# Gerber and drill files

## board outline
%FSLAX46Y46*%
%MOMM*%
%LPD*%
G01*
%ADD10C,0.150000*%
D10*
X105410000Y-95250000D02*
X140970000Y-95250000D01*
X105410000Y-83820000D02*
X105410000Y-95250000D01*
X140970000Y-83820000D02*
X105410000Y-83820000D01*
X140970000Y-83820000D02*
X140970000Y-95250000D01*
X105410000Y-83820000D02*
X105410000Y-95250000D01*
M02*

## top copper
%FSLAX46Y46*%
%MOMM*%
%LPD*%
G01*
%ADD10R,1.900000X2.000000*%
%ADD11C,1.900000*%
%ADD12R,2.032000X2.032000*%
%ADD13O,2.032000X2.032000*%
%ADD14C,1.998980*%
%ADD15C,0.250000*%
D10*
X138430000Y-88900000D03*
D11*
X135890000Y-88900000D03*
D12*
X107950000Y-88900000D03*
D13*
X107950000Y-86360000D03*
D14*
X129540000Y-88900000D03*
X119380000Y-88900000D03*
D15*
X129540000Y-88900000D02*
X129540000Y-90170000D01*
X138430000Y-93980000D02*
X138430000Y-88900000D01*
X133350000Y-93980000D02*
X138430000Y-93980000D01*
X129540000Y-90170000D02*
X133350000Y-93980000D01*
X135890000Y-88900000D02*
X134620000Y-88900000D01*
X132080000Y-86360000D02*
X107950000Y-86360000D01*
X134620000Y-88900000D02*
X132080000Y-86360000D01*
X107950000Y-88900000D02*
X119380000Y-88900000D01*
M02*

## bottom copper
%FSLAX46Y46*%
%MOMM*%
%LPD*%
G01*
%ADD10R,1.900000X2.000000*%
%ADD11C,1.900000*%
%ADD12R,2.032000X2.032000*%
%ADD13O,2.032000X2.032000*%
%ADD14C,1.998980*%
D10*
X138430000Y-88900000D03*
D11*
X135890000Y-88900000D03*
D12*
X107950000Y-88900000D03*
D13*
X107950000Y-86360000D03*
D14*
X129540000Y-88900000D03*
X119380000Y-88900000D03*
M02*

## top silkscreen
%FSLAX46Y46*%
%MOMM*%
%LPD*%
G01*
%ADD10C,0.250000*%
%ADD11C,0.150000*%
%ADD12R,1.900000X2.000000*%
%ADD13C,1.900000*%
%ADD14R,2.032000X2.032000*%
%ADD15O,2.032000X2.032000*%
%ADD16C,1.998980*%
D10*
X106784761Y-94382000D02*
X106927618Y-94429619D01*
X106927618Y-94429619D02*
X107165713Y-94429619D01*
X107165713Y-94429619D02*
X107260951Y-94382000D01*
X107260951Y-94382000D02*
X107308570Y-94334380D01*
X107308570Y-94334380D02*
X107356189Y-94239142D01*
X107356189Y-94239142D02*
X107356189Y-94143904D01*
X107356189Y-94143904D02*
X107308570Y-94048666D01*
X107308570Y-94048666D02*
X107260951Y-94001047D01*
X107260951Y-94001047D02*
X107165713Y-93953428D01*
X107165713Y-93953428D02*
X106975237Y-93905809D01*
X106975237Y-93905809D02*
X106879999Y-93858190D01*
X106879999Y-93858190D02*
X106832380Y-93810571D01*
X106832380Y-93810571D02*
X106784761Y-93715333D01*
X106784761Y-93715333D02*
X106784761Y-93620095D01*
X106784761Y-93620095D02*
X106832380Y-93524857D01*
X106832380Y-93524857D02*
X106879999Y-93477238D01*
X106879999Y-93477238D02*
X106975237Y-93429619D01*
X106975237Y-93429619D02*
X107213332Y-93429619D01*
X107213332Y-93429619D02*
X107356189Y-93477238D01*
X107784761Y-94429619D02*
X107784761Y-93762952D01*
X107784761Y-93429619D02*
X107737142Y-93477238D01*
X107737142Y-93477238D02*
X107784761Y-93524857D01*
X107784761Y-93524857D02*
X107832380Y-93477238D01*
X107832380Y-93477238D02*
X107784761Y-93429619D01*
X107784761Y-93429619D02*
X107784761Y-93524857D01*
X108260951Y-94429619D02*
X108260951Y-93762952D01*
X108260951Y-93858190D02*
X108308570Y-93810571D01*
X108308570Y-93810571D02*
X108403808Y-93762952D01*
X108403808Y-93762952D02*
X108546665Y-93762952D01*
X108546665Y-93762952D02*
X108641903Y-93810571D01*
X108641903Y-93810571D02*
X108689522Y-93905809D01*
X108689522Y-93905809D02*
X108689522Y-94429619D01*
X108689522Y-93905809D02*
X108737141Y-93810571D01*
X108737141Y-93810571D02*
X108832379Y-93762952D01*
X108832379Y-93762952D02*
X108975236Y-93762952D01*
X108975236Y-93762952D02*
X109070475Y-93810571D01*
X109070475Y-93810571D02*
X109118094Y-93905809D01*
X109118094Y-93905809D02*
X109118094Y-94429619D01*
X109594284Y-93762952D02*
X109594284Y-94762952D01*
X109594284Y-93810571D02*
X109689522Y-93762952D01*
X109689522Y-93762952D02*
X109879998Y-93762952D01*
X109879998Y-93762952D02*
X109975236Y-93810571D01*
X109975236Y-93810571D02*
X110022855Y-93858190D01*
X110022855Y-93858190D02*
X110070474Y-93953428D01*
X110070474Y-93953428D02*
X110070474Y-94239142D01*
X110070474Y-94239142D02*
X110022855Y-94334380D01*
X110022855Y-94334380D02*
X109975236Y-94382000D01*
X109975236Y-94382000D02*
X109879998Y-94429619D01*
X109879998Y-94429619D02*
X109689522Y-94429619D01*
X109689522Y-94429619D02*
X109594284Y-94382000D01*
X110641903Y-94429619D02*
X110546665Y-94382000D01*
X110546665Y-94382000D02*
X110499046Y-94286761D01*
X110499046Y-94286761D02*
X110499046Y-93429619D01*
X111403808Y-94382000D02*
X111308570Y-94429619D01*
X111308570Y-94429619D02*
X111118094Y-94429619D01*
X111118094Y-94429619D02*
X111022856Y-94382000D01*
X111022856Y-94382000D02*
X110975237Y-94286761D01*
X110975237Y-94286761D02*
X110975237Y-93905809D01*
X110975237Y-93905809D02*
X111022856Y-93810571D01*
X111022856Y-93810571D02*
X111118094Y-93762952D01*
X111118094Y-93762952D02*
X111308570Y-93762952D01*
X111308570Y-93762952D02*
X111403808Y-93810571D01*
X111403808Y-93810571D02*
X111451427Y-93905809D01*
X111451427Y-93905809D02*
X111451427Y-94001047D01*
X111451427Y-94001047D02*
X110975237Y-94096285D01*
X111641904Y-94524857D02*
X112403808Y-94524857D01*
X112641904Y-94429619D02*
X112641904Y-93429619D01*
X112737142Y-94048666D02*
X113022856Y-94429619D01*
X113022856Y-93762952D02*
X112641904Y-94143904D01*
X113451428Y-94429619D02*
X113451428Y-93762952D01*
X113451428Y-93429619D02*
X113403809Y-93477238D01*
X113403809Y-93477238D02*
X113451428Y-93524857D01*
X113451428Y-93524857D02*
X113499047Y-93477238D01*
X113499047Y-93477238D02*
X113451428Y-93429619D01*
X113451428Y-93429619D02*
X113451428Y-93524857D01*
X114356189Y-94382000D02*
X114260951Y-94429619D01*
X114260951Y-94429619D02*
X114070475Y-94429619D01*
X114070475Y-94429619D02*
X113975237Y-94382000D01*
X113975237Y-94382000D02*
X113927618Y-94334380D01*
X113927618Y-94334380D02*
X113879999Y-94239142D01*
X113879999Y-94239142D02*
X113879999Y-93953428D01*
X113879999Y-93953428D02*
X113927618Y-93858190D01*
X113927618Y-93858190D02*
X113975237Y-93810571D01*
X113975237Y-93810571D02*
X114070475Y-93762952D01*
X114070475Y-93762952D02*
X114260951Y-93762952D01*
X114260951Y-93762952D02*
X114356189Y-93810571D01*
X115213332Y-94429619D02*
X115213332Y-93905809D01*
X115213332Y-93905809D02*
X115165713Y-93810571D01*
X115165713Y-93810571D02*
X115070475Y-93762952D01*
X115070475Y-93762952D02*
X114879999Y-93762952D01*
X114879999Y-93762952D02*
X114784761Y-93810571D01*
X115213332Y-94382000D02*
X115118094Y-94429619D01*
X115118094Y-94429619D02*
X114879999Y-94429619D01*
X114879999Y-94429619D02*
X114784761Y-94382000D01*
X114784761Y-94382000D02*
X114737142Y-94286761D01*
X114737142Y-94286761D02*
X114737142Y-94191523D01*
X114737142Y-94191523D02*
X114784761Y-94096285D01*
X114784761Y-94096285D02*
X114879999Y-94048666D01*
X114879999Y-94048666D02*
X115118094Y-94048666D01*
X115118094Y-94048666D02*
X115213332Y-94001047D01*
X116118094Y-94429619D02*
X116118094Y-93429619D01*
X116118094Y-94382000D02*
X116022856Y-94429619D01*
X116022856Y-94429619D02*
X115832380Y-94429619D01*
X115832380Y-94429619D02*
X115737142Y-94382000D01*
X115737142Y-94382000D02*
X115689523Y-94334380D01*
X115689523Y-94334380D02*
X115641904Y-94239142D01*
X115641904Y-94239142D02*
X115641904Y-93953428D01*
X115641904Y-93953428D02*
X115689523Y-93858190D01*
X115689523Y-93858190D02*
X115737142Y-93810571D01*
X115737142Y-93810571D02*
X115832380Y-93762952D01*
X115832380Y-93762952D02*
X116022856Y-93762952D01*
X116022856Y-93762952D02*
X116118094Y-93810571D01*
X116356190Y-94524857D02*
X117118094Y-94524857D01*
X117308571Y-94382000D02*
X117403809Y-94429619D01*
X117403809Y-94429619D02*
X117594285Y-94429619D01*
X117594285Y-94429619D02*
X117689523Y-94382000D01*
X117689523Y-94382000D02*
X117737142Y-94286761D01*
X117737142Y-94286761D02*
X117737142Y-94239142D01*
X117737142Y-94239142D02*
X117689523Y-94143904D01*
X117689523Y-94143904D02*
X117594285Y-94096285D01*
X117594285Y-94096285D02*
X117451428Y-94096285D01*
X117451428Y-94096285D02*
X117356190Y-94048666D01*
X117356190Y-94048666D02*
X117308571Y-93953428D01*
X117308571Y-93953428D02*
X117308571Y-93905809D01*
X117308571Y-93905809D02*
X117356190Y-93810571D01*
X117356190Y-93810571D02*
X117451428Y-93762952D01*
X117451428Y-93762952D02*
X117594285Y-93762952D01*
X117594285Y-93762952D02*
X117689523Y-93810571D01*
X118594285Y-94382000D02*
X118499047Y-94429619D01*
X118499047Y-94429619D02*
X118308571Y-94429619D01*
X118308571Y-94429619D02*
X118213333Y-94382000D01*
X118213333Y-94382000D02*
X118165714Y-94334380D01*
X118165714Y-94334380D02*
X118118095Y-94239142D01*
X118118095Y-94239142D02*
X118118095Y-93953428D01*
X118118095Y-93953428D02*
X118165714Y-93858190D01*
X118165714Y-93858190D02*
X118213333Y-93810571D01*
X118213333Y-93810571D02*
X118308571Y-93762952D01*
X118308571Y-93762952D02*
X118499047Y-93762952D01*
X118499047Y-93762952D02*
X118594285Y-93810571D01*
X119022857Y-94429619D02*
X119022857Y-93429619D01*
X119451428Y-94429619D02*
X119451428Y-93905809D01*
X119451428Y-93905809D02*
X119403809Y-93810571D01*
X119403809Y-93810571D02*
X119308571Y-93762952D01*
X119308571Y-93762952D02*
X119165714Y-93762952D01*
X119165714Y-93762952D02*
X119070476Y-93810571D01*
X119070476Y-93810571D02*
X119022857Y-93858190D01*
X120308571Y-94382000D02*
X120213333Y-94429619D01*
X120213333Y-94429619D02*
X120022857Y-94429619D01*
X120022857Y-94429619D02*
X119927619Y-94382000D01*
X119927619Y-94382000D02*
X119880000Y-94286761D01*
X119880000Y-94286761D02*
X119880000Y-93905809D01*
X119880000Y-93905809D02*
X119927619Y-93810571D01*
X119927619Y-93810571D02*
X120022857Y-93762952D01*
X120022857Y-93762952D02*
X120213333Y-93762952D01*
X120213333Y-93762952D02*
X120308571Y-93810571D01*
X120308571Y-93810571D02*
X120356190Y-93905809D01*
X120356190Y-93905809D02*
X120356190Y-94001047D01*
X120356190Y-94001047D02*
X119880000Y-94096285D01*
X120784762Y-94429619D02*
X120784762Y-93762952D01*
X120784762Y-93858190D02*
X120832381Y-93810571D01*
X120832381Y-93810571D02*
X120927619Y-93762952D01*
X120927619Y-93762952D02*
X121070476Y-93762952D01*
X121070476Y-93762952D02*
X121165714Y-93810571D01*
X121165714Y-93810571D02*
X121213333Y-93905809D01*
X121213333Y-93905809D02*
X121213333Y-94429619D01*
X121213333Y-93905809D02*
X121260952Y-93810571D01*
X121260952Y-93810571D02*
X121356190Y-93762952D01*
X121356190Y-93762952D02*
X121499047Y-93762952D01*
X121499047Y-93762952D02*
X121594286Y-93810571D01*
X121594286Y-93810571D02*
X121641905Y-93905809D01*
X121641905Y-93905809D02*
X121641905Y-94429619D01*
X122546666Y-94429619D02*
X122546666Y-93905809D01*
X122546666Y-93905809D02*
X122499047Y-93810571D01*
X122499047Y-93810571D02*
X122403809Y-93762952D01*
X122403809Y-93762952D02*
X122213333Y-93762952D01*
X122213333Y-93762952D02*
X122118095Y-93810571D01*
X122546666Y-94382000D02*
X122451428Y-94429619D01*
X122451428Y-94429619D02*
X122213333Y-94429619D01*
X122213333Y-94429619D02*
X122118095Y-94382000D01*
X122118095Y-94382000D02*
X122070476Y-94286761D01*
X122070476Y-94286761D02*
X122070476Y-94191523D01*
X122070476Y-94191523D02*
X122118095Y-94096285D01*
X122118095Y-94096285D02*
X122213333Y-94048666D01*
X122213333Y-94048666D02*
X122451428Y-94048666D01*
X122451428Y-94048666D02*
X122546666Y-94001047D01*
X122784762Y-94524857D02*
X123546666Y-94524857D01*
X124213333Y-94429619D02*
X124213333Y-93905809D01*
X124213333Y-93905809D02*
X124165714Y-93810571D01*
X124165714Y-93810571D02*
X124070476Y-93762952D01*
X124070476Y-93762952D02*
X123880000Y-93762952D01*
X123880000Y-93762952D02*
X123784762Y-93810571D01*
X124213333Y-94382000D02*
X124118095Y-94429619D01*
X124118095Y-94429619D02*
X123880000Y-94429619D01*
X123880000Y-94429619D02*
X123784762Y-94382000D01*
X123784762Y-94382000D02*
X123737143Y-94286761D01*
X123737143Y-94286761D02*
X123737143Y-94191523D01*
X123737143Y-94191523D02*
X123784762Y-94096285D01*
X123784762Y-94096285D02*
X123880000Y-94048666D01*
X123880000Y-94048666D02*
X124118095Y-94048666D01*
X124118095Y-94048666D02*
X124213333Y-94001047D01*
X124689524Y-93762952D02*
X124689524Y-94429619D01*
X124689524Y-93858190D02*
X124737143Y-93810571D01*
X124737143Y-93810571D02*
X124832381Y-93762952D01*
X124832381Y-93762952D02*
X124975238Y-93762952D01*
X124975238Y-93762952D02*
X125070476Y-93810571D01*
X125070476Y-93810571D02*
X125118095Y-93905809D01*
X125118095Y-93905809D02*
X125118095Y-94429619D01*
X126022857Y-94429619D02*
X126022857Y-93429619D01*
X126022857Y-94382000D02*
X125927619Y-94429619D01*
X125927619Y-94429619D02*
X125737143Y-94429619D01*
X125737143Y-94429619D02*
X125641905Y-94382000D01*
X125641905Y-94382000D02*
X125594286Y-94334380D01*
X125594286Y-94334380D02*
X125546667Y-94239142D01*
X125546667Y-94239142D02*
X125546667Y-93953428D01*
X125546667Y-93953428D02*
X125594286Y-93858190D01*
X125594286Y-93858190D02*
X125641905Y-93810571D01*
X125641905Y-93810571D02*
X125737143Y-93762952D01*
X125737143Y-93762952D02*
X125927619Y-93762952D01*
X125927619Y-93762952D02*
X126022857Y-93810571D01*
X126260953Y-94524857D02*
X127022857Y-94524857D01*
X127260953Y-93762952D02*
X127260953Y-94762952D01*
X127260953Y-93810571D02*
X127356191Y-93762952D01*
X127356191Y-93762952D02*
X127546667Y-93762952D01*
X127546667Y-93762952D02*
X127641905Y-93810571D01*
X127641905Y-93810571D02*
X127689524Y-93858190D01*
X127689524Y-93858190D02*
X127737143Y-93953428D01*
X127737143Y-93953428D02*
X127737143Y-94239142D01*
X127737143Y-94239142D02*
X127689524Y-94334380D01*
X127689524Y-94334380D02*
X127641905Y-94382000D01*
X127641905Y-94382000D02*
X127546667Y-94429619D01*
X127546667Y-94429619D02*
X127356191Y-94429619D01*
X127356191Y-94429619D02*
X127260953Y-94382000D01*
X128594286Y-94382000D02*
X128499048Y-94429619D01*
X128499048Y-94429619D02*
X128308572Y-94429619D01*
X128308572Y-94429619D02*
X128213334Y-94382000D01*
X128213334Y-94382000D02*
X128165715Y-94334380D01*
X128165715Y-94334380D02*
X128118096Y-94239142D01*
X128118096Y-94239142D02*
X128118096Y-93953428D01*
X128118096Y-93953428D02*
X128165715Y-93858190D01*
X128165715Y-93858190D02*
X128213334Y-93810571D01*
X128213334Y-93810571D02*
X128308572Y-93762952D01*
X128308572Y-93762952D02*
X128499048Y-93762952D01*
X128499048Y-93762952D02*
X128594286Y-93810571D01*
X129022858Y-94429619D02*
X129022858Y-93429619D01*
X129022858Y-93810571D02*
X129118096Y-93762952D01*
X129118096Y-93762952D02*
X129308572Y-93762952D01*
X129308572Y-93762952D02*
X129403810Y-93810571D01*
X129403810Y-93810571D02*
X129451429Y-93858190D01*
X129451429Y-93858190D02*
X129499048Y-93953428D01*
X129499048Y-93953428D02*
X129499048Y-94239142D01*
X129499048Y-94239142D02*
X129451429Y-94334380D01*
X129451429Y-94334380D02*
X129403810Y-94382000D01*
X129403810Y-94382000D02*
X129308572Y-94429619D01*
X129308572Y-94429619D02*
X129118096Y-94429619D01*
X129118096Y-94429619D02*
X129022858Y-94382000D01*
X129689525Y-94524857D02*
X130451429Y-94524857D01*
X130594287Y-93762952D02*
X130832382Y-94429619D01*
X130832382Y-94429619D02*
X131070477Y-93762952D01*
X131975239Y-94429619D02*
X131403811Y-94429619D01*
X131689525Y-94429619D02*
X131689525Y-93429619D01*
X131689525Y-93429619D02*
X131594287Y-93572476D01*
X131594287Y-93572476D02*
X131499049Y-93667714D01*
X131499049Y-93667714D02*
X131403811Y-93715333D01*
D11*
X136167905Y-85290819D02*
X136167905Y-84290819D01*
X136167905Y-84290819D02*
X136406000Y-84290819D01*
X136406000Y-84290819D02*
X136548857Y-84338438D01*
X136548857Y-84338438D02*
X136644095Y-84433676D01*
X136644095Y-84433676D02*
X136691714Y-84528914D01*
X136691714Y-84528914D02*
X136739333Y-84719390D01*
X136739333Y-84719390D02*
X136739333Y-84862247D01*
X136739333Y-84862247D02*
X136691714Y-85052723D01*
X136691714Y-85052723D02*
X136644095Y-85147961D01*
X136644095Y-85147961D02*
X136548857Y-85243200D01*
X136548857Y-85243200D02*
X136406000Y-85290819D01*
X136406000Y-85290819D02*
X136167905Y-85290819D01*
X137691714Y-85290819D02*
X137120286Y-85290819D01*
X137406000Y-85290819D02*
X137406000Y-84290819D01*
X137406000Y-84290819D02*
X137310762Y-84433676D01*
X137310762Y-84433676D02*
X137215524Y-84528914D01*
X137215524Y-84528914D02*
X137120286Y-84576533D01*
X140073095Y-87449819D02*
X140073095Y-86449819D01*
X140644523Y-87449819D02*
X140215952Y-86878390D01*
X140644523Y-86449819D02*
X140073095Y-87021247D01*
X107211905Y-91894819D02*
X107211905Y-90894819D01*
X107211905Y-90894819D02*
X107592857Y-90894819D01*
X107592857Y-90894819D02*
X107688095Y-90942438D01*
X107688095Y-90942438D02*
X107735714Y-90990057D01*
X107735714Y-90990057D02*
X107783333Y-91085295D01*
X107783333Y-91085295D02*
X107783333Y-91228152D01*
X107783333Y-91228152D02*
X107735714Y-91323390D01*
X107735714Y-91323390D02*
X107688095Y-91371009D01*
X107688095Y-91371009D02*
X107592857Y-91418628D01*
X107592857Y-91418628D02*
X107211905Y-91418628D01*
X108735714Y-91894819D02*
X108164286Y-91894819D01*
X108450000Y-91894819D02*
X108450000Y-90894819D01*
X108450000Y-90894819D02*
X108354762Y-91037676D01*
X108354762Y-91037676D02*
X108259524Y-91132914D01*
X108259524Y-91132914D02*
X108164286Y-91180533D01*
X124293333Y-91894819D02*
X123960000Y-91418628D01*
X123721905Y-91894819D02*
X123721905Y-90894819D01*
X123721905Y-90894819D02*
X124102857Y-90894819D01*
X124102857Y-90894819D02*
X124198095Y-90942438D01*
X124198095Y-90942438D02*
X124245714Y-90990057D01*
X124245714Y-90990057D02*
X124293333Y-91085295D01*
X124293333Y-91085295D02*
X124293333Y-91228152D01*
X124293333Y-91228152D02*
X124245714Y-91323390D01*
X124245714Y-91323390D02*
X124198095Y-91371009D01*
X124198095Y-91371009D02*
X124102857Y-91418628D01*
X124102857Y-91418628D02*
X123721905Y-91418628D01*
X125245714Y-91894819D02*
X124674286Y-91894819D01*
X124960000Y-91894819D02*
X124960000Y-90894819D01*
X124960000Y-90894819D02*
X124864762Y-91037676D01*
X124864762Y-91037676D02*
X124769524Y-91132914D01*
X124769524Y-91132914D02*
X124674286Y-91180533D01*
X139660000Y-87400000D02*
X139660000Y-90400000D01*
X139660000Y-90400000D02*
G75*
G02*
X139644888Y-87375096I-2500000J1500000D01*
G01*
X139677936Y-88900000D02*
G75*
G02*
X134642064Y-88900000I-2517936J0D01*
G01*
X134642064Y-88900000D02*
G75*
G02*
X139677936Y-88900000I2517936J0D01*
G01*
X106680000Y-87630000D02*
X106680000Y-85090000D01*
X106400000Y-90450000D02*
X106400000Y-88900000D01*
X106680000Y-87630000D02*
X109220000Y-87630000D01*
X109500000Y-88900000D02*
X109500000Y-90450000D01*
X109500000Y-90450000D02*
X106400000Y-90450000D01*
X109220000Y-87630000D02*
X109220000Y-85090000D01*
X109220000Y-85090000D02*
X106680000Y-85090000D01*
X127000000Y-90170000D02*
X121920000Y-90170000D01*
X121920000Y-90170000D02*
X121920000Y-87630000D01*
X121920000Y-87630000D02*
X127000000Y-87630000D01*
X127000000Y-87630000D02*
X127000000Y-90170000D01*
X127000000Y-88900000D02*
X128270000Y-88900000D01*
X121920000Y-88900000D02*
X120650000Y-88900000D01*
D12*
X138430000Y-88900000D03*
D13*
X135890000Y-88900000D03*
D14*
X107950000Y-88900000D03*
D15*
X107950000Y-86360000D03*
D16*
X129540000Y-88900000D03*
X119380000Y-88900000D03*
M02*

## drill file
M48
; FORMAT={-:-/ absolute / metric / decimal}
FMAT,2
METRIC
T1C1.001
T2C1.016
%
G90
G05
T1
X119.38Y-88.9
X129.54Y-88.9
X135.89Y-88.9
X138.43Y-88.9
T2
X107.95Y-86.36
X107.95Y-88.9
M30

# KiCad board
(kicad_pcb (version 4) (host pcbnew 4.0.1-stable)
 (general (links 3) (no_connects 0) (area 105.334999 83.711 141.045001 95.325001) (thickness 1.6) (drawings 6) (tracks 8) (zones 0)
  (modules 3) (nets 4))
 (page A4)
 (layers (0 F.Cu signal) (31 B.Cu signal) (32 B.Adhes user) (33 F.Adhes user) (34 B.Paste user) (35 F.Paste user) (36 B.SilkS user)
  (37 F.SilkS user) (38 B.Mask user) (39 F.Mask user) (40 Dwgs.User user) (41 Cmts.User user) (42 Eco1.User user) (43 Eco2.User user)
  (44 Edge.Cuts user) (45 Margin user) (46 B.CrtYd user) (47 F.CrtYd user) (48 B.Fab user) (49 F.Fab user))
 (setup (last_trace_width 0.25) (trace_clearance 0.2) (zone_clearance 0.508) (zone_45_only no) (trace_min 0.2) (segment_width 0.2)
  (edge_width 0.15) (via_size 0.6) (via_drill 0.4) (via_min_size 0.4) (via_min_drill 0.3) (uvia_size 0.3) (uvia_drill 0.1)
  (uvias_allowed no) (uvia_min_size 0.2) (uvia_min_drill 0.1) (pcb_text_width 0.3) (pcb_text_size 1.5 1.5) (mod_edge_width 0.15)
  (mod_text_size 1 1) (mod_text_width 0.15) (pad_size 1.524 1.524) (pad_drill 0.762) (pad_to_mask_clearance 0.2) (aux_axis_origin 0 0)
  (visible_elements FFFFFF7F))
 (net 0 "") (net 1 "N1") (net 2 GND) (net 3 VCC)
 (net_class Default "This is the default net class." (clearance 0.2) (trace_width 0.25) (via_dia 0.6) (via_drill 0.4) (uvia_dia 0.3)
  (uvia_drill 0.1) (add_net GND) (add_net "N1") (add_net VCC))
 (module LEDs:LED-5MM (layer F.Cu) (at 138.43 88.9 180)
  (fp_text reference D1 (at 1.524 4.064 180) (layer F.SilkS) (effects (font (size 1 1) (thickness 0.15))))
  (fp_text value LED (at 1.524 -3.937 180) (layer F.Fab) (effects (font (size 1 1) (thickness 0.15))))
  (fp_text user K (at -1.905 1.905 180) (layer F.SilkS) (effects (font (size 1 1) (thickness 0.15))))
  (fp_line (start -1.23 1.5) (end -1.23 -1.5) (layer F.SilkS) (width 0.15))
  (fp_arc (start 1.27 0) (end -1.23 -1.5) (angle 297.5) (layer F.SilkS) (width 0.15))
  (fp_circle (center 1.27 0) (end 0.97 -2.5) (layer F.SilkS) (width 0.15))
  (pad 1 thru_hole rect (at 0 0 270) (size 2 1.9) (drill 1.00076) (layers *.Cu *.Mask F.SilkS) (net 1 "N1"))
  (pad 2 thru_hole circle (at 2.54 0 180) (size 1.9 1.9) (drill 1.00076) (layers *.Cu *.Mask F.SilkS) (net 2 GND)))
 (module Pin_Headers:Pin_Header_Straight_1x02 (layer F.Cu) (at 107.95 88.9 180)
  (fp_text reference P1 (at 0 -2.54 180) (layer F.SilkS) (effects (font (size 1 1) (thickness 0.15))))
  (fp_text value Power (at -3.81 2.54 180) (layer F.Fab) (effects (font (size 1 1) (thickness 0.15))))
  (fp_line (start 1.27 1.27) (end 1.27 3.81) (layer F.SilkS) (width 0.15))
  (fp_line (start 1.55 -1.55) (end 1.55 0) (layer F.SilkS) (width 0.15))
  (fp_line (start 1.27 1.27) (end -1.27 1.27) (layer F.SilkS) (width 0.15))
  (fp_line (start -1.55 0) (end -1.55 -1.55) (layer F.SilkS) (width 0.15))
  (fp_line (start -1.55 -1.55) (end 1.55 -1.55) (layer F.SilkS) (width 0.15))
  (fp_line (start -1.27 1.27) (end -1.27 3.81) (layer F.SilkS) (width 0.15))
  (fp_line (start -1.27 3.81) (end 1.27 3.81) (layer F.SilkS) (width 0.15))
  (pad 1 thru_hole rect (at 0 0 180) (size 2.032 2.032) (drill 1.016) (layers *.Cu *.Mask F.SilkS) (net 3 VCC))
  (pad 2 thru_hole oval (at 0 2.54 180) (size 2.032 2.032) (drill 1.016) (layers *.Cu *.Mask F.SilkS) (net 2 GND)))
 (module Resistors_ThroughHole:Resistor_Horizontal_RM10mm (layer F.Cu) (at 124.46 88.9 180)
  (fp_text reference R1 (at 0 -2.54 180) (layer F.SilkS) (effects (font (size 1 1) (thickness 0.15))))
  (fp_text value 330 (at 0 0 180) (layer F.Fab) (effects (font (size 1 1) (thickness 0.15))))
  (fp_line (start -2.54 -1.27) (end 2.54 -1.27) (layer F.SilkS) (width 0.15))
  (fp_line (start 2.54 -1.27) (end 2.54 1.27) (layer F.SilkS) (width 0.15))
  (fp_line (start 2.54 1.27) (end -2.54 1.27) (layer F.SilkS) (width 0.15))
  (fp_line (start -2.54 1.27) (end -2.54 -1.27) (layer F.SilkS) (width 0.15))
  (fp_line (start -2.54 0) (end -3.81 0) (layer F.SilkS) (width 0.15))
  (fp_line (start 2.54 0) (end 3.81 0) (layer F.SilkS) (width 0.15))
  (pad 1 thru_hole circle (at -5.08 0 180) (size 1.99898 1.99898) (drill 1.00076) (layers *.Cu *.SilkS *.Mask) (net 1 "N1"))
  (pad 2 thru_hole circle (at 5.08 0 180) (size 1.99898 1.99898) (drill 1.00076) (layers *.Cu *.SilkS *.Mask) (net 3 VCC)))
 (gr_line (start 105.41 95.25) (end 140.97 95.25) (angle 90) (layer Edge.Cuts) (width 0.15))
 (gr_line (start 105.41 83.82) (end 105.41 95.25) (angle 90) (layer Edge.Cuts) (width 0.15))
 (gr_line (start 140.97 83.82) (end 105.41 83.82) (angle 90) (layer Edge.Cuts) (width 0.15))
 (gr_line (start 140.97 83.82) (end 140.97 95.25) (angle 90) (layer Edge.Cuts) (width 0.15))
 (gr_line (start 105.41 83.82) (end 105.41 95.25) (angle 90) (layer Edge.Cuts) (width 0.15))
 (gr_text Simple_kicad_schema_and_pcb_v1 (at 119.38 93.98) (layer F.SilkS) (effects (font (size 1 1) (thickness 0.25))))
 (segment (start 129.54 88.9) (end 129.54 90.17) (width 0.25) (layer F.Cu) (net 1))
 (segment (start 138.43 93.98) (end 138.43 88.9) (width 0.25) (layer F.Cu) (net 1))
 (segment (start 133.35 93.98) (end 138.43 93.98) (width 0.25) (layer F.Cu) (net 1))
 (segment (start 129.54 90.17) (end 133.35 93.98) (width 0.25) (layer F.Cu) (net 1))
 (segment (start 135.89 88.9) (end 134.62 88.9) (width 0.25) (layer F.Cu) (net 2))
 (segment (start 132.08 86.36) (end 107.95 86.36) (width 0.25) (layer F.Cu) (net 2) (status 20))
 (segment (start 134.62 88.9) (end 132.08 86.36) (width 0.25) (layer F.Cu) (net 2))
 (segment (start 107.95 88.9) (end 119.38 88.9) (width 0.25) (layer F.Cu) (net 3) (status 10)))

